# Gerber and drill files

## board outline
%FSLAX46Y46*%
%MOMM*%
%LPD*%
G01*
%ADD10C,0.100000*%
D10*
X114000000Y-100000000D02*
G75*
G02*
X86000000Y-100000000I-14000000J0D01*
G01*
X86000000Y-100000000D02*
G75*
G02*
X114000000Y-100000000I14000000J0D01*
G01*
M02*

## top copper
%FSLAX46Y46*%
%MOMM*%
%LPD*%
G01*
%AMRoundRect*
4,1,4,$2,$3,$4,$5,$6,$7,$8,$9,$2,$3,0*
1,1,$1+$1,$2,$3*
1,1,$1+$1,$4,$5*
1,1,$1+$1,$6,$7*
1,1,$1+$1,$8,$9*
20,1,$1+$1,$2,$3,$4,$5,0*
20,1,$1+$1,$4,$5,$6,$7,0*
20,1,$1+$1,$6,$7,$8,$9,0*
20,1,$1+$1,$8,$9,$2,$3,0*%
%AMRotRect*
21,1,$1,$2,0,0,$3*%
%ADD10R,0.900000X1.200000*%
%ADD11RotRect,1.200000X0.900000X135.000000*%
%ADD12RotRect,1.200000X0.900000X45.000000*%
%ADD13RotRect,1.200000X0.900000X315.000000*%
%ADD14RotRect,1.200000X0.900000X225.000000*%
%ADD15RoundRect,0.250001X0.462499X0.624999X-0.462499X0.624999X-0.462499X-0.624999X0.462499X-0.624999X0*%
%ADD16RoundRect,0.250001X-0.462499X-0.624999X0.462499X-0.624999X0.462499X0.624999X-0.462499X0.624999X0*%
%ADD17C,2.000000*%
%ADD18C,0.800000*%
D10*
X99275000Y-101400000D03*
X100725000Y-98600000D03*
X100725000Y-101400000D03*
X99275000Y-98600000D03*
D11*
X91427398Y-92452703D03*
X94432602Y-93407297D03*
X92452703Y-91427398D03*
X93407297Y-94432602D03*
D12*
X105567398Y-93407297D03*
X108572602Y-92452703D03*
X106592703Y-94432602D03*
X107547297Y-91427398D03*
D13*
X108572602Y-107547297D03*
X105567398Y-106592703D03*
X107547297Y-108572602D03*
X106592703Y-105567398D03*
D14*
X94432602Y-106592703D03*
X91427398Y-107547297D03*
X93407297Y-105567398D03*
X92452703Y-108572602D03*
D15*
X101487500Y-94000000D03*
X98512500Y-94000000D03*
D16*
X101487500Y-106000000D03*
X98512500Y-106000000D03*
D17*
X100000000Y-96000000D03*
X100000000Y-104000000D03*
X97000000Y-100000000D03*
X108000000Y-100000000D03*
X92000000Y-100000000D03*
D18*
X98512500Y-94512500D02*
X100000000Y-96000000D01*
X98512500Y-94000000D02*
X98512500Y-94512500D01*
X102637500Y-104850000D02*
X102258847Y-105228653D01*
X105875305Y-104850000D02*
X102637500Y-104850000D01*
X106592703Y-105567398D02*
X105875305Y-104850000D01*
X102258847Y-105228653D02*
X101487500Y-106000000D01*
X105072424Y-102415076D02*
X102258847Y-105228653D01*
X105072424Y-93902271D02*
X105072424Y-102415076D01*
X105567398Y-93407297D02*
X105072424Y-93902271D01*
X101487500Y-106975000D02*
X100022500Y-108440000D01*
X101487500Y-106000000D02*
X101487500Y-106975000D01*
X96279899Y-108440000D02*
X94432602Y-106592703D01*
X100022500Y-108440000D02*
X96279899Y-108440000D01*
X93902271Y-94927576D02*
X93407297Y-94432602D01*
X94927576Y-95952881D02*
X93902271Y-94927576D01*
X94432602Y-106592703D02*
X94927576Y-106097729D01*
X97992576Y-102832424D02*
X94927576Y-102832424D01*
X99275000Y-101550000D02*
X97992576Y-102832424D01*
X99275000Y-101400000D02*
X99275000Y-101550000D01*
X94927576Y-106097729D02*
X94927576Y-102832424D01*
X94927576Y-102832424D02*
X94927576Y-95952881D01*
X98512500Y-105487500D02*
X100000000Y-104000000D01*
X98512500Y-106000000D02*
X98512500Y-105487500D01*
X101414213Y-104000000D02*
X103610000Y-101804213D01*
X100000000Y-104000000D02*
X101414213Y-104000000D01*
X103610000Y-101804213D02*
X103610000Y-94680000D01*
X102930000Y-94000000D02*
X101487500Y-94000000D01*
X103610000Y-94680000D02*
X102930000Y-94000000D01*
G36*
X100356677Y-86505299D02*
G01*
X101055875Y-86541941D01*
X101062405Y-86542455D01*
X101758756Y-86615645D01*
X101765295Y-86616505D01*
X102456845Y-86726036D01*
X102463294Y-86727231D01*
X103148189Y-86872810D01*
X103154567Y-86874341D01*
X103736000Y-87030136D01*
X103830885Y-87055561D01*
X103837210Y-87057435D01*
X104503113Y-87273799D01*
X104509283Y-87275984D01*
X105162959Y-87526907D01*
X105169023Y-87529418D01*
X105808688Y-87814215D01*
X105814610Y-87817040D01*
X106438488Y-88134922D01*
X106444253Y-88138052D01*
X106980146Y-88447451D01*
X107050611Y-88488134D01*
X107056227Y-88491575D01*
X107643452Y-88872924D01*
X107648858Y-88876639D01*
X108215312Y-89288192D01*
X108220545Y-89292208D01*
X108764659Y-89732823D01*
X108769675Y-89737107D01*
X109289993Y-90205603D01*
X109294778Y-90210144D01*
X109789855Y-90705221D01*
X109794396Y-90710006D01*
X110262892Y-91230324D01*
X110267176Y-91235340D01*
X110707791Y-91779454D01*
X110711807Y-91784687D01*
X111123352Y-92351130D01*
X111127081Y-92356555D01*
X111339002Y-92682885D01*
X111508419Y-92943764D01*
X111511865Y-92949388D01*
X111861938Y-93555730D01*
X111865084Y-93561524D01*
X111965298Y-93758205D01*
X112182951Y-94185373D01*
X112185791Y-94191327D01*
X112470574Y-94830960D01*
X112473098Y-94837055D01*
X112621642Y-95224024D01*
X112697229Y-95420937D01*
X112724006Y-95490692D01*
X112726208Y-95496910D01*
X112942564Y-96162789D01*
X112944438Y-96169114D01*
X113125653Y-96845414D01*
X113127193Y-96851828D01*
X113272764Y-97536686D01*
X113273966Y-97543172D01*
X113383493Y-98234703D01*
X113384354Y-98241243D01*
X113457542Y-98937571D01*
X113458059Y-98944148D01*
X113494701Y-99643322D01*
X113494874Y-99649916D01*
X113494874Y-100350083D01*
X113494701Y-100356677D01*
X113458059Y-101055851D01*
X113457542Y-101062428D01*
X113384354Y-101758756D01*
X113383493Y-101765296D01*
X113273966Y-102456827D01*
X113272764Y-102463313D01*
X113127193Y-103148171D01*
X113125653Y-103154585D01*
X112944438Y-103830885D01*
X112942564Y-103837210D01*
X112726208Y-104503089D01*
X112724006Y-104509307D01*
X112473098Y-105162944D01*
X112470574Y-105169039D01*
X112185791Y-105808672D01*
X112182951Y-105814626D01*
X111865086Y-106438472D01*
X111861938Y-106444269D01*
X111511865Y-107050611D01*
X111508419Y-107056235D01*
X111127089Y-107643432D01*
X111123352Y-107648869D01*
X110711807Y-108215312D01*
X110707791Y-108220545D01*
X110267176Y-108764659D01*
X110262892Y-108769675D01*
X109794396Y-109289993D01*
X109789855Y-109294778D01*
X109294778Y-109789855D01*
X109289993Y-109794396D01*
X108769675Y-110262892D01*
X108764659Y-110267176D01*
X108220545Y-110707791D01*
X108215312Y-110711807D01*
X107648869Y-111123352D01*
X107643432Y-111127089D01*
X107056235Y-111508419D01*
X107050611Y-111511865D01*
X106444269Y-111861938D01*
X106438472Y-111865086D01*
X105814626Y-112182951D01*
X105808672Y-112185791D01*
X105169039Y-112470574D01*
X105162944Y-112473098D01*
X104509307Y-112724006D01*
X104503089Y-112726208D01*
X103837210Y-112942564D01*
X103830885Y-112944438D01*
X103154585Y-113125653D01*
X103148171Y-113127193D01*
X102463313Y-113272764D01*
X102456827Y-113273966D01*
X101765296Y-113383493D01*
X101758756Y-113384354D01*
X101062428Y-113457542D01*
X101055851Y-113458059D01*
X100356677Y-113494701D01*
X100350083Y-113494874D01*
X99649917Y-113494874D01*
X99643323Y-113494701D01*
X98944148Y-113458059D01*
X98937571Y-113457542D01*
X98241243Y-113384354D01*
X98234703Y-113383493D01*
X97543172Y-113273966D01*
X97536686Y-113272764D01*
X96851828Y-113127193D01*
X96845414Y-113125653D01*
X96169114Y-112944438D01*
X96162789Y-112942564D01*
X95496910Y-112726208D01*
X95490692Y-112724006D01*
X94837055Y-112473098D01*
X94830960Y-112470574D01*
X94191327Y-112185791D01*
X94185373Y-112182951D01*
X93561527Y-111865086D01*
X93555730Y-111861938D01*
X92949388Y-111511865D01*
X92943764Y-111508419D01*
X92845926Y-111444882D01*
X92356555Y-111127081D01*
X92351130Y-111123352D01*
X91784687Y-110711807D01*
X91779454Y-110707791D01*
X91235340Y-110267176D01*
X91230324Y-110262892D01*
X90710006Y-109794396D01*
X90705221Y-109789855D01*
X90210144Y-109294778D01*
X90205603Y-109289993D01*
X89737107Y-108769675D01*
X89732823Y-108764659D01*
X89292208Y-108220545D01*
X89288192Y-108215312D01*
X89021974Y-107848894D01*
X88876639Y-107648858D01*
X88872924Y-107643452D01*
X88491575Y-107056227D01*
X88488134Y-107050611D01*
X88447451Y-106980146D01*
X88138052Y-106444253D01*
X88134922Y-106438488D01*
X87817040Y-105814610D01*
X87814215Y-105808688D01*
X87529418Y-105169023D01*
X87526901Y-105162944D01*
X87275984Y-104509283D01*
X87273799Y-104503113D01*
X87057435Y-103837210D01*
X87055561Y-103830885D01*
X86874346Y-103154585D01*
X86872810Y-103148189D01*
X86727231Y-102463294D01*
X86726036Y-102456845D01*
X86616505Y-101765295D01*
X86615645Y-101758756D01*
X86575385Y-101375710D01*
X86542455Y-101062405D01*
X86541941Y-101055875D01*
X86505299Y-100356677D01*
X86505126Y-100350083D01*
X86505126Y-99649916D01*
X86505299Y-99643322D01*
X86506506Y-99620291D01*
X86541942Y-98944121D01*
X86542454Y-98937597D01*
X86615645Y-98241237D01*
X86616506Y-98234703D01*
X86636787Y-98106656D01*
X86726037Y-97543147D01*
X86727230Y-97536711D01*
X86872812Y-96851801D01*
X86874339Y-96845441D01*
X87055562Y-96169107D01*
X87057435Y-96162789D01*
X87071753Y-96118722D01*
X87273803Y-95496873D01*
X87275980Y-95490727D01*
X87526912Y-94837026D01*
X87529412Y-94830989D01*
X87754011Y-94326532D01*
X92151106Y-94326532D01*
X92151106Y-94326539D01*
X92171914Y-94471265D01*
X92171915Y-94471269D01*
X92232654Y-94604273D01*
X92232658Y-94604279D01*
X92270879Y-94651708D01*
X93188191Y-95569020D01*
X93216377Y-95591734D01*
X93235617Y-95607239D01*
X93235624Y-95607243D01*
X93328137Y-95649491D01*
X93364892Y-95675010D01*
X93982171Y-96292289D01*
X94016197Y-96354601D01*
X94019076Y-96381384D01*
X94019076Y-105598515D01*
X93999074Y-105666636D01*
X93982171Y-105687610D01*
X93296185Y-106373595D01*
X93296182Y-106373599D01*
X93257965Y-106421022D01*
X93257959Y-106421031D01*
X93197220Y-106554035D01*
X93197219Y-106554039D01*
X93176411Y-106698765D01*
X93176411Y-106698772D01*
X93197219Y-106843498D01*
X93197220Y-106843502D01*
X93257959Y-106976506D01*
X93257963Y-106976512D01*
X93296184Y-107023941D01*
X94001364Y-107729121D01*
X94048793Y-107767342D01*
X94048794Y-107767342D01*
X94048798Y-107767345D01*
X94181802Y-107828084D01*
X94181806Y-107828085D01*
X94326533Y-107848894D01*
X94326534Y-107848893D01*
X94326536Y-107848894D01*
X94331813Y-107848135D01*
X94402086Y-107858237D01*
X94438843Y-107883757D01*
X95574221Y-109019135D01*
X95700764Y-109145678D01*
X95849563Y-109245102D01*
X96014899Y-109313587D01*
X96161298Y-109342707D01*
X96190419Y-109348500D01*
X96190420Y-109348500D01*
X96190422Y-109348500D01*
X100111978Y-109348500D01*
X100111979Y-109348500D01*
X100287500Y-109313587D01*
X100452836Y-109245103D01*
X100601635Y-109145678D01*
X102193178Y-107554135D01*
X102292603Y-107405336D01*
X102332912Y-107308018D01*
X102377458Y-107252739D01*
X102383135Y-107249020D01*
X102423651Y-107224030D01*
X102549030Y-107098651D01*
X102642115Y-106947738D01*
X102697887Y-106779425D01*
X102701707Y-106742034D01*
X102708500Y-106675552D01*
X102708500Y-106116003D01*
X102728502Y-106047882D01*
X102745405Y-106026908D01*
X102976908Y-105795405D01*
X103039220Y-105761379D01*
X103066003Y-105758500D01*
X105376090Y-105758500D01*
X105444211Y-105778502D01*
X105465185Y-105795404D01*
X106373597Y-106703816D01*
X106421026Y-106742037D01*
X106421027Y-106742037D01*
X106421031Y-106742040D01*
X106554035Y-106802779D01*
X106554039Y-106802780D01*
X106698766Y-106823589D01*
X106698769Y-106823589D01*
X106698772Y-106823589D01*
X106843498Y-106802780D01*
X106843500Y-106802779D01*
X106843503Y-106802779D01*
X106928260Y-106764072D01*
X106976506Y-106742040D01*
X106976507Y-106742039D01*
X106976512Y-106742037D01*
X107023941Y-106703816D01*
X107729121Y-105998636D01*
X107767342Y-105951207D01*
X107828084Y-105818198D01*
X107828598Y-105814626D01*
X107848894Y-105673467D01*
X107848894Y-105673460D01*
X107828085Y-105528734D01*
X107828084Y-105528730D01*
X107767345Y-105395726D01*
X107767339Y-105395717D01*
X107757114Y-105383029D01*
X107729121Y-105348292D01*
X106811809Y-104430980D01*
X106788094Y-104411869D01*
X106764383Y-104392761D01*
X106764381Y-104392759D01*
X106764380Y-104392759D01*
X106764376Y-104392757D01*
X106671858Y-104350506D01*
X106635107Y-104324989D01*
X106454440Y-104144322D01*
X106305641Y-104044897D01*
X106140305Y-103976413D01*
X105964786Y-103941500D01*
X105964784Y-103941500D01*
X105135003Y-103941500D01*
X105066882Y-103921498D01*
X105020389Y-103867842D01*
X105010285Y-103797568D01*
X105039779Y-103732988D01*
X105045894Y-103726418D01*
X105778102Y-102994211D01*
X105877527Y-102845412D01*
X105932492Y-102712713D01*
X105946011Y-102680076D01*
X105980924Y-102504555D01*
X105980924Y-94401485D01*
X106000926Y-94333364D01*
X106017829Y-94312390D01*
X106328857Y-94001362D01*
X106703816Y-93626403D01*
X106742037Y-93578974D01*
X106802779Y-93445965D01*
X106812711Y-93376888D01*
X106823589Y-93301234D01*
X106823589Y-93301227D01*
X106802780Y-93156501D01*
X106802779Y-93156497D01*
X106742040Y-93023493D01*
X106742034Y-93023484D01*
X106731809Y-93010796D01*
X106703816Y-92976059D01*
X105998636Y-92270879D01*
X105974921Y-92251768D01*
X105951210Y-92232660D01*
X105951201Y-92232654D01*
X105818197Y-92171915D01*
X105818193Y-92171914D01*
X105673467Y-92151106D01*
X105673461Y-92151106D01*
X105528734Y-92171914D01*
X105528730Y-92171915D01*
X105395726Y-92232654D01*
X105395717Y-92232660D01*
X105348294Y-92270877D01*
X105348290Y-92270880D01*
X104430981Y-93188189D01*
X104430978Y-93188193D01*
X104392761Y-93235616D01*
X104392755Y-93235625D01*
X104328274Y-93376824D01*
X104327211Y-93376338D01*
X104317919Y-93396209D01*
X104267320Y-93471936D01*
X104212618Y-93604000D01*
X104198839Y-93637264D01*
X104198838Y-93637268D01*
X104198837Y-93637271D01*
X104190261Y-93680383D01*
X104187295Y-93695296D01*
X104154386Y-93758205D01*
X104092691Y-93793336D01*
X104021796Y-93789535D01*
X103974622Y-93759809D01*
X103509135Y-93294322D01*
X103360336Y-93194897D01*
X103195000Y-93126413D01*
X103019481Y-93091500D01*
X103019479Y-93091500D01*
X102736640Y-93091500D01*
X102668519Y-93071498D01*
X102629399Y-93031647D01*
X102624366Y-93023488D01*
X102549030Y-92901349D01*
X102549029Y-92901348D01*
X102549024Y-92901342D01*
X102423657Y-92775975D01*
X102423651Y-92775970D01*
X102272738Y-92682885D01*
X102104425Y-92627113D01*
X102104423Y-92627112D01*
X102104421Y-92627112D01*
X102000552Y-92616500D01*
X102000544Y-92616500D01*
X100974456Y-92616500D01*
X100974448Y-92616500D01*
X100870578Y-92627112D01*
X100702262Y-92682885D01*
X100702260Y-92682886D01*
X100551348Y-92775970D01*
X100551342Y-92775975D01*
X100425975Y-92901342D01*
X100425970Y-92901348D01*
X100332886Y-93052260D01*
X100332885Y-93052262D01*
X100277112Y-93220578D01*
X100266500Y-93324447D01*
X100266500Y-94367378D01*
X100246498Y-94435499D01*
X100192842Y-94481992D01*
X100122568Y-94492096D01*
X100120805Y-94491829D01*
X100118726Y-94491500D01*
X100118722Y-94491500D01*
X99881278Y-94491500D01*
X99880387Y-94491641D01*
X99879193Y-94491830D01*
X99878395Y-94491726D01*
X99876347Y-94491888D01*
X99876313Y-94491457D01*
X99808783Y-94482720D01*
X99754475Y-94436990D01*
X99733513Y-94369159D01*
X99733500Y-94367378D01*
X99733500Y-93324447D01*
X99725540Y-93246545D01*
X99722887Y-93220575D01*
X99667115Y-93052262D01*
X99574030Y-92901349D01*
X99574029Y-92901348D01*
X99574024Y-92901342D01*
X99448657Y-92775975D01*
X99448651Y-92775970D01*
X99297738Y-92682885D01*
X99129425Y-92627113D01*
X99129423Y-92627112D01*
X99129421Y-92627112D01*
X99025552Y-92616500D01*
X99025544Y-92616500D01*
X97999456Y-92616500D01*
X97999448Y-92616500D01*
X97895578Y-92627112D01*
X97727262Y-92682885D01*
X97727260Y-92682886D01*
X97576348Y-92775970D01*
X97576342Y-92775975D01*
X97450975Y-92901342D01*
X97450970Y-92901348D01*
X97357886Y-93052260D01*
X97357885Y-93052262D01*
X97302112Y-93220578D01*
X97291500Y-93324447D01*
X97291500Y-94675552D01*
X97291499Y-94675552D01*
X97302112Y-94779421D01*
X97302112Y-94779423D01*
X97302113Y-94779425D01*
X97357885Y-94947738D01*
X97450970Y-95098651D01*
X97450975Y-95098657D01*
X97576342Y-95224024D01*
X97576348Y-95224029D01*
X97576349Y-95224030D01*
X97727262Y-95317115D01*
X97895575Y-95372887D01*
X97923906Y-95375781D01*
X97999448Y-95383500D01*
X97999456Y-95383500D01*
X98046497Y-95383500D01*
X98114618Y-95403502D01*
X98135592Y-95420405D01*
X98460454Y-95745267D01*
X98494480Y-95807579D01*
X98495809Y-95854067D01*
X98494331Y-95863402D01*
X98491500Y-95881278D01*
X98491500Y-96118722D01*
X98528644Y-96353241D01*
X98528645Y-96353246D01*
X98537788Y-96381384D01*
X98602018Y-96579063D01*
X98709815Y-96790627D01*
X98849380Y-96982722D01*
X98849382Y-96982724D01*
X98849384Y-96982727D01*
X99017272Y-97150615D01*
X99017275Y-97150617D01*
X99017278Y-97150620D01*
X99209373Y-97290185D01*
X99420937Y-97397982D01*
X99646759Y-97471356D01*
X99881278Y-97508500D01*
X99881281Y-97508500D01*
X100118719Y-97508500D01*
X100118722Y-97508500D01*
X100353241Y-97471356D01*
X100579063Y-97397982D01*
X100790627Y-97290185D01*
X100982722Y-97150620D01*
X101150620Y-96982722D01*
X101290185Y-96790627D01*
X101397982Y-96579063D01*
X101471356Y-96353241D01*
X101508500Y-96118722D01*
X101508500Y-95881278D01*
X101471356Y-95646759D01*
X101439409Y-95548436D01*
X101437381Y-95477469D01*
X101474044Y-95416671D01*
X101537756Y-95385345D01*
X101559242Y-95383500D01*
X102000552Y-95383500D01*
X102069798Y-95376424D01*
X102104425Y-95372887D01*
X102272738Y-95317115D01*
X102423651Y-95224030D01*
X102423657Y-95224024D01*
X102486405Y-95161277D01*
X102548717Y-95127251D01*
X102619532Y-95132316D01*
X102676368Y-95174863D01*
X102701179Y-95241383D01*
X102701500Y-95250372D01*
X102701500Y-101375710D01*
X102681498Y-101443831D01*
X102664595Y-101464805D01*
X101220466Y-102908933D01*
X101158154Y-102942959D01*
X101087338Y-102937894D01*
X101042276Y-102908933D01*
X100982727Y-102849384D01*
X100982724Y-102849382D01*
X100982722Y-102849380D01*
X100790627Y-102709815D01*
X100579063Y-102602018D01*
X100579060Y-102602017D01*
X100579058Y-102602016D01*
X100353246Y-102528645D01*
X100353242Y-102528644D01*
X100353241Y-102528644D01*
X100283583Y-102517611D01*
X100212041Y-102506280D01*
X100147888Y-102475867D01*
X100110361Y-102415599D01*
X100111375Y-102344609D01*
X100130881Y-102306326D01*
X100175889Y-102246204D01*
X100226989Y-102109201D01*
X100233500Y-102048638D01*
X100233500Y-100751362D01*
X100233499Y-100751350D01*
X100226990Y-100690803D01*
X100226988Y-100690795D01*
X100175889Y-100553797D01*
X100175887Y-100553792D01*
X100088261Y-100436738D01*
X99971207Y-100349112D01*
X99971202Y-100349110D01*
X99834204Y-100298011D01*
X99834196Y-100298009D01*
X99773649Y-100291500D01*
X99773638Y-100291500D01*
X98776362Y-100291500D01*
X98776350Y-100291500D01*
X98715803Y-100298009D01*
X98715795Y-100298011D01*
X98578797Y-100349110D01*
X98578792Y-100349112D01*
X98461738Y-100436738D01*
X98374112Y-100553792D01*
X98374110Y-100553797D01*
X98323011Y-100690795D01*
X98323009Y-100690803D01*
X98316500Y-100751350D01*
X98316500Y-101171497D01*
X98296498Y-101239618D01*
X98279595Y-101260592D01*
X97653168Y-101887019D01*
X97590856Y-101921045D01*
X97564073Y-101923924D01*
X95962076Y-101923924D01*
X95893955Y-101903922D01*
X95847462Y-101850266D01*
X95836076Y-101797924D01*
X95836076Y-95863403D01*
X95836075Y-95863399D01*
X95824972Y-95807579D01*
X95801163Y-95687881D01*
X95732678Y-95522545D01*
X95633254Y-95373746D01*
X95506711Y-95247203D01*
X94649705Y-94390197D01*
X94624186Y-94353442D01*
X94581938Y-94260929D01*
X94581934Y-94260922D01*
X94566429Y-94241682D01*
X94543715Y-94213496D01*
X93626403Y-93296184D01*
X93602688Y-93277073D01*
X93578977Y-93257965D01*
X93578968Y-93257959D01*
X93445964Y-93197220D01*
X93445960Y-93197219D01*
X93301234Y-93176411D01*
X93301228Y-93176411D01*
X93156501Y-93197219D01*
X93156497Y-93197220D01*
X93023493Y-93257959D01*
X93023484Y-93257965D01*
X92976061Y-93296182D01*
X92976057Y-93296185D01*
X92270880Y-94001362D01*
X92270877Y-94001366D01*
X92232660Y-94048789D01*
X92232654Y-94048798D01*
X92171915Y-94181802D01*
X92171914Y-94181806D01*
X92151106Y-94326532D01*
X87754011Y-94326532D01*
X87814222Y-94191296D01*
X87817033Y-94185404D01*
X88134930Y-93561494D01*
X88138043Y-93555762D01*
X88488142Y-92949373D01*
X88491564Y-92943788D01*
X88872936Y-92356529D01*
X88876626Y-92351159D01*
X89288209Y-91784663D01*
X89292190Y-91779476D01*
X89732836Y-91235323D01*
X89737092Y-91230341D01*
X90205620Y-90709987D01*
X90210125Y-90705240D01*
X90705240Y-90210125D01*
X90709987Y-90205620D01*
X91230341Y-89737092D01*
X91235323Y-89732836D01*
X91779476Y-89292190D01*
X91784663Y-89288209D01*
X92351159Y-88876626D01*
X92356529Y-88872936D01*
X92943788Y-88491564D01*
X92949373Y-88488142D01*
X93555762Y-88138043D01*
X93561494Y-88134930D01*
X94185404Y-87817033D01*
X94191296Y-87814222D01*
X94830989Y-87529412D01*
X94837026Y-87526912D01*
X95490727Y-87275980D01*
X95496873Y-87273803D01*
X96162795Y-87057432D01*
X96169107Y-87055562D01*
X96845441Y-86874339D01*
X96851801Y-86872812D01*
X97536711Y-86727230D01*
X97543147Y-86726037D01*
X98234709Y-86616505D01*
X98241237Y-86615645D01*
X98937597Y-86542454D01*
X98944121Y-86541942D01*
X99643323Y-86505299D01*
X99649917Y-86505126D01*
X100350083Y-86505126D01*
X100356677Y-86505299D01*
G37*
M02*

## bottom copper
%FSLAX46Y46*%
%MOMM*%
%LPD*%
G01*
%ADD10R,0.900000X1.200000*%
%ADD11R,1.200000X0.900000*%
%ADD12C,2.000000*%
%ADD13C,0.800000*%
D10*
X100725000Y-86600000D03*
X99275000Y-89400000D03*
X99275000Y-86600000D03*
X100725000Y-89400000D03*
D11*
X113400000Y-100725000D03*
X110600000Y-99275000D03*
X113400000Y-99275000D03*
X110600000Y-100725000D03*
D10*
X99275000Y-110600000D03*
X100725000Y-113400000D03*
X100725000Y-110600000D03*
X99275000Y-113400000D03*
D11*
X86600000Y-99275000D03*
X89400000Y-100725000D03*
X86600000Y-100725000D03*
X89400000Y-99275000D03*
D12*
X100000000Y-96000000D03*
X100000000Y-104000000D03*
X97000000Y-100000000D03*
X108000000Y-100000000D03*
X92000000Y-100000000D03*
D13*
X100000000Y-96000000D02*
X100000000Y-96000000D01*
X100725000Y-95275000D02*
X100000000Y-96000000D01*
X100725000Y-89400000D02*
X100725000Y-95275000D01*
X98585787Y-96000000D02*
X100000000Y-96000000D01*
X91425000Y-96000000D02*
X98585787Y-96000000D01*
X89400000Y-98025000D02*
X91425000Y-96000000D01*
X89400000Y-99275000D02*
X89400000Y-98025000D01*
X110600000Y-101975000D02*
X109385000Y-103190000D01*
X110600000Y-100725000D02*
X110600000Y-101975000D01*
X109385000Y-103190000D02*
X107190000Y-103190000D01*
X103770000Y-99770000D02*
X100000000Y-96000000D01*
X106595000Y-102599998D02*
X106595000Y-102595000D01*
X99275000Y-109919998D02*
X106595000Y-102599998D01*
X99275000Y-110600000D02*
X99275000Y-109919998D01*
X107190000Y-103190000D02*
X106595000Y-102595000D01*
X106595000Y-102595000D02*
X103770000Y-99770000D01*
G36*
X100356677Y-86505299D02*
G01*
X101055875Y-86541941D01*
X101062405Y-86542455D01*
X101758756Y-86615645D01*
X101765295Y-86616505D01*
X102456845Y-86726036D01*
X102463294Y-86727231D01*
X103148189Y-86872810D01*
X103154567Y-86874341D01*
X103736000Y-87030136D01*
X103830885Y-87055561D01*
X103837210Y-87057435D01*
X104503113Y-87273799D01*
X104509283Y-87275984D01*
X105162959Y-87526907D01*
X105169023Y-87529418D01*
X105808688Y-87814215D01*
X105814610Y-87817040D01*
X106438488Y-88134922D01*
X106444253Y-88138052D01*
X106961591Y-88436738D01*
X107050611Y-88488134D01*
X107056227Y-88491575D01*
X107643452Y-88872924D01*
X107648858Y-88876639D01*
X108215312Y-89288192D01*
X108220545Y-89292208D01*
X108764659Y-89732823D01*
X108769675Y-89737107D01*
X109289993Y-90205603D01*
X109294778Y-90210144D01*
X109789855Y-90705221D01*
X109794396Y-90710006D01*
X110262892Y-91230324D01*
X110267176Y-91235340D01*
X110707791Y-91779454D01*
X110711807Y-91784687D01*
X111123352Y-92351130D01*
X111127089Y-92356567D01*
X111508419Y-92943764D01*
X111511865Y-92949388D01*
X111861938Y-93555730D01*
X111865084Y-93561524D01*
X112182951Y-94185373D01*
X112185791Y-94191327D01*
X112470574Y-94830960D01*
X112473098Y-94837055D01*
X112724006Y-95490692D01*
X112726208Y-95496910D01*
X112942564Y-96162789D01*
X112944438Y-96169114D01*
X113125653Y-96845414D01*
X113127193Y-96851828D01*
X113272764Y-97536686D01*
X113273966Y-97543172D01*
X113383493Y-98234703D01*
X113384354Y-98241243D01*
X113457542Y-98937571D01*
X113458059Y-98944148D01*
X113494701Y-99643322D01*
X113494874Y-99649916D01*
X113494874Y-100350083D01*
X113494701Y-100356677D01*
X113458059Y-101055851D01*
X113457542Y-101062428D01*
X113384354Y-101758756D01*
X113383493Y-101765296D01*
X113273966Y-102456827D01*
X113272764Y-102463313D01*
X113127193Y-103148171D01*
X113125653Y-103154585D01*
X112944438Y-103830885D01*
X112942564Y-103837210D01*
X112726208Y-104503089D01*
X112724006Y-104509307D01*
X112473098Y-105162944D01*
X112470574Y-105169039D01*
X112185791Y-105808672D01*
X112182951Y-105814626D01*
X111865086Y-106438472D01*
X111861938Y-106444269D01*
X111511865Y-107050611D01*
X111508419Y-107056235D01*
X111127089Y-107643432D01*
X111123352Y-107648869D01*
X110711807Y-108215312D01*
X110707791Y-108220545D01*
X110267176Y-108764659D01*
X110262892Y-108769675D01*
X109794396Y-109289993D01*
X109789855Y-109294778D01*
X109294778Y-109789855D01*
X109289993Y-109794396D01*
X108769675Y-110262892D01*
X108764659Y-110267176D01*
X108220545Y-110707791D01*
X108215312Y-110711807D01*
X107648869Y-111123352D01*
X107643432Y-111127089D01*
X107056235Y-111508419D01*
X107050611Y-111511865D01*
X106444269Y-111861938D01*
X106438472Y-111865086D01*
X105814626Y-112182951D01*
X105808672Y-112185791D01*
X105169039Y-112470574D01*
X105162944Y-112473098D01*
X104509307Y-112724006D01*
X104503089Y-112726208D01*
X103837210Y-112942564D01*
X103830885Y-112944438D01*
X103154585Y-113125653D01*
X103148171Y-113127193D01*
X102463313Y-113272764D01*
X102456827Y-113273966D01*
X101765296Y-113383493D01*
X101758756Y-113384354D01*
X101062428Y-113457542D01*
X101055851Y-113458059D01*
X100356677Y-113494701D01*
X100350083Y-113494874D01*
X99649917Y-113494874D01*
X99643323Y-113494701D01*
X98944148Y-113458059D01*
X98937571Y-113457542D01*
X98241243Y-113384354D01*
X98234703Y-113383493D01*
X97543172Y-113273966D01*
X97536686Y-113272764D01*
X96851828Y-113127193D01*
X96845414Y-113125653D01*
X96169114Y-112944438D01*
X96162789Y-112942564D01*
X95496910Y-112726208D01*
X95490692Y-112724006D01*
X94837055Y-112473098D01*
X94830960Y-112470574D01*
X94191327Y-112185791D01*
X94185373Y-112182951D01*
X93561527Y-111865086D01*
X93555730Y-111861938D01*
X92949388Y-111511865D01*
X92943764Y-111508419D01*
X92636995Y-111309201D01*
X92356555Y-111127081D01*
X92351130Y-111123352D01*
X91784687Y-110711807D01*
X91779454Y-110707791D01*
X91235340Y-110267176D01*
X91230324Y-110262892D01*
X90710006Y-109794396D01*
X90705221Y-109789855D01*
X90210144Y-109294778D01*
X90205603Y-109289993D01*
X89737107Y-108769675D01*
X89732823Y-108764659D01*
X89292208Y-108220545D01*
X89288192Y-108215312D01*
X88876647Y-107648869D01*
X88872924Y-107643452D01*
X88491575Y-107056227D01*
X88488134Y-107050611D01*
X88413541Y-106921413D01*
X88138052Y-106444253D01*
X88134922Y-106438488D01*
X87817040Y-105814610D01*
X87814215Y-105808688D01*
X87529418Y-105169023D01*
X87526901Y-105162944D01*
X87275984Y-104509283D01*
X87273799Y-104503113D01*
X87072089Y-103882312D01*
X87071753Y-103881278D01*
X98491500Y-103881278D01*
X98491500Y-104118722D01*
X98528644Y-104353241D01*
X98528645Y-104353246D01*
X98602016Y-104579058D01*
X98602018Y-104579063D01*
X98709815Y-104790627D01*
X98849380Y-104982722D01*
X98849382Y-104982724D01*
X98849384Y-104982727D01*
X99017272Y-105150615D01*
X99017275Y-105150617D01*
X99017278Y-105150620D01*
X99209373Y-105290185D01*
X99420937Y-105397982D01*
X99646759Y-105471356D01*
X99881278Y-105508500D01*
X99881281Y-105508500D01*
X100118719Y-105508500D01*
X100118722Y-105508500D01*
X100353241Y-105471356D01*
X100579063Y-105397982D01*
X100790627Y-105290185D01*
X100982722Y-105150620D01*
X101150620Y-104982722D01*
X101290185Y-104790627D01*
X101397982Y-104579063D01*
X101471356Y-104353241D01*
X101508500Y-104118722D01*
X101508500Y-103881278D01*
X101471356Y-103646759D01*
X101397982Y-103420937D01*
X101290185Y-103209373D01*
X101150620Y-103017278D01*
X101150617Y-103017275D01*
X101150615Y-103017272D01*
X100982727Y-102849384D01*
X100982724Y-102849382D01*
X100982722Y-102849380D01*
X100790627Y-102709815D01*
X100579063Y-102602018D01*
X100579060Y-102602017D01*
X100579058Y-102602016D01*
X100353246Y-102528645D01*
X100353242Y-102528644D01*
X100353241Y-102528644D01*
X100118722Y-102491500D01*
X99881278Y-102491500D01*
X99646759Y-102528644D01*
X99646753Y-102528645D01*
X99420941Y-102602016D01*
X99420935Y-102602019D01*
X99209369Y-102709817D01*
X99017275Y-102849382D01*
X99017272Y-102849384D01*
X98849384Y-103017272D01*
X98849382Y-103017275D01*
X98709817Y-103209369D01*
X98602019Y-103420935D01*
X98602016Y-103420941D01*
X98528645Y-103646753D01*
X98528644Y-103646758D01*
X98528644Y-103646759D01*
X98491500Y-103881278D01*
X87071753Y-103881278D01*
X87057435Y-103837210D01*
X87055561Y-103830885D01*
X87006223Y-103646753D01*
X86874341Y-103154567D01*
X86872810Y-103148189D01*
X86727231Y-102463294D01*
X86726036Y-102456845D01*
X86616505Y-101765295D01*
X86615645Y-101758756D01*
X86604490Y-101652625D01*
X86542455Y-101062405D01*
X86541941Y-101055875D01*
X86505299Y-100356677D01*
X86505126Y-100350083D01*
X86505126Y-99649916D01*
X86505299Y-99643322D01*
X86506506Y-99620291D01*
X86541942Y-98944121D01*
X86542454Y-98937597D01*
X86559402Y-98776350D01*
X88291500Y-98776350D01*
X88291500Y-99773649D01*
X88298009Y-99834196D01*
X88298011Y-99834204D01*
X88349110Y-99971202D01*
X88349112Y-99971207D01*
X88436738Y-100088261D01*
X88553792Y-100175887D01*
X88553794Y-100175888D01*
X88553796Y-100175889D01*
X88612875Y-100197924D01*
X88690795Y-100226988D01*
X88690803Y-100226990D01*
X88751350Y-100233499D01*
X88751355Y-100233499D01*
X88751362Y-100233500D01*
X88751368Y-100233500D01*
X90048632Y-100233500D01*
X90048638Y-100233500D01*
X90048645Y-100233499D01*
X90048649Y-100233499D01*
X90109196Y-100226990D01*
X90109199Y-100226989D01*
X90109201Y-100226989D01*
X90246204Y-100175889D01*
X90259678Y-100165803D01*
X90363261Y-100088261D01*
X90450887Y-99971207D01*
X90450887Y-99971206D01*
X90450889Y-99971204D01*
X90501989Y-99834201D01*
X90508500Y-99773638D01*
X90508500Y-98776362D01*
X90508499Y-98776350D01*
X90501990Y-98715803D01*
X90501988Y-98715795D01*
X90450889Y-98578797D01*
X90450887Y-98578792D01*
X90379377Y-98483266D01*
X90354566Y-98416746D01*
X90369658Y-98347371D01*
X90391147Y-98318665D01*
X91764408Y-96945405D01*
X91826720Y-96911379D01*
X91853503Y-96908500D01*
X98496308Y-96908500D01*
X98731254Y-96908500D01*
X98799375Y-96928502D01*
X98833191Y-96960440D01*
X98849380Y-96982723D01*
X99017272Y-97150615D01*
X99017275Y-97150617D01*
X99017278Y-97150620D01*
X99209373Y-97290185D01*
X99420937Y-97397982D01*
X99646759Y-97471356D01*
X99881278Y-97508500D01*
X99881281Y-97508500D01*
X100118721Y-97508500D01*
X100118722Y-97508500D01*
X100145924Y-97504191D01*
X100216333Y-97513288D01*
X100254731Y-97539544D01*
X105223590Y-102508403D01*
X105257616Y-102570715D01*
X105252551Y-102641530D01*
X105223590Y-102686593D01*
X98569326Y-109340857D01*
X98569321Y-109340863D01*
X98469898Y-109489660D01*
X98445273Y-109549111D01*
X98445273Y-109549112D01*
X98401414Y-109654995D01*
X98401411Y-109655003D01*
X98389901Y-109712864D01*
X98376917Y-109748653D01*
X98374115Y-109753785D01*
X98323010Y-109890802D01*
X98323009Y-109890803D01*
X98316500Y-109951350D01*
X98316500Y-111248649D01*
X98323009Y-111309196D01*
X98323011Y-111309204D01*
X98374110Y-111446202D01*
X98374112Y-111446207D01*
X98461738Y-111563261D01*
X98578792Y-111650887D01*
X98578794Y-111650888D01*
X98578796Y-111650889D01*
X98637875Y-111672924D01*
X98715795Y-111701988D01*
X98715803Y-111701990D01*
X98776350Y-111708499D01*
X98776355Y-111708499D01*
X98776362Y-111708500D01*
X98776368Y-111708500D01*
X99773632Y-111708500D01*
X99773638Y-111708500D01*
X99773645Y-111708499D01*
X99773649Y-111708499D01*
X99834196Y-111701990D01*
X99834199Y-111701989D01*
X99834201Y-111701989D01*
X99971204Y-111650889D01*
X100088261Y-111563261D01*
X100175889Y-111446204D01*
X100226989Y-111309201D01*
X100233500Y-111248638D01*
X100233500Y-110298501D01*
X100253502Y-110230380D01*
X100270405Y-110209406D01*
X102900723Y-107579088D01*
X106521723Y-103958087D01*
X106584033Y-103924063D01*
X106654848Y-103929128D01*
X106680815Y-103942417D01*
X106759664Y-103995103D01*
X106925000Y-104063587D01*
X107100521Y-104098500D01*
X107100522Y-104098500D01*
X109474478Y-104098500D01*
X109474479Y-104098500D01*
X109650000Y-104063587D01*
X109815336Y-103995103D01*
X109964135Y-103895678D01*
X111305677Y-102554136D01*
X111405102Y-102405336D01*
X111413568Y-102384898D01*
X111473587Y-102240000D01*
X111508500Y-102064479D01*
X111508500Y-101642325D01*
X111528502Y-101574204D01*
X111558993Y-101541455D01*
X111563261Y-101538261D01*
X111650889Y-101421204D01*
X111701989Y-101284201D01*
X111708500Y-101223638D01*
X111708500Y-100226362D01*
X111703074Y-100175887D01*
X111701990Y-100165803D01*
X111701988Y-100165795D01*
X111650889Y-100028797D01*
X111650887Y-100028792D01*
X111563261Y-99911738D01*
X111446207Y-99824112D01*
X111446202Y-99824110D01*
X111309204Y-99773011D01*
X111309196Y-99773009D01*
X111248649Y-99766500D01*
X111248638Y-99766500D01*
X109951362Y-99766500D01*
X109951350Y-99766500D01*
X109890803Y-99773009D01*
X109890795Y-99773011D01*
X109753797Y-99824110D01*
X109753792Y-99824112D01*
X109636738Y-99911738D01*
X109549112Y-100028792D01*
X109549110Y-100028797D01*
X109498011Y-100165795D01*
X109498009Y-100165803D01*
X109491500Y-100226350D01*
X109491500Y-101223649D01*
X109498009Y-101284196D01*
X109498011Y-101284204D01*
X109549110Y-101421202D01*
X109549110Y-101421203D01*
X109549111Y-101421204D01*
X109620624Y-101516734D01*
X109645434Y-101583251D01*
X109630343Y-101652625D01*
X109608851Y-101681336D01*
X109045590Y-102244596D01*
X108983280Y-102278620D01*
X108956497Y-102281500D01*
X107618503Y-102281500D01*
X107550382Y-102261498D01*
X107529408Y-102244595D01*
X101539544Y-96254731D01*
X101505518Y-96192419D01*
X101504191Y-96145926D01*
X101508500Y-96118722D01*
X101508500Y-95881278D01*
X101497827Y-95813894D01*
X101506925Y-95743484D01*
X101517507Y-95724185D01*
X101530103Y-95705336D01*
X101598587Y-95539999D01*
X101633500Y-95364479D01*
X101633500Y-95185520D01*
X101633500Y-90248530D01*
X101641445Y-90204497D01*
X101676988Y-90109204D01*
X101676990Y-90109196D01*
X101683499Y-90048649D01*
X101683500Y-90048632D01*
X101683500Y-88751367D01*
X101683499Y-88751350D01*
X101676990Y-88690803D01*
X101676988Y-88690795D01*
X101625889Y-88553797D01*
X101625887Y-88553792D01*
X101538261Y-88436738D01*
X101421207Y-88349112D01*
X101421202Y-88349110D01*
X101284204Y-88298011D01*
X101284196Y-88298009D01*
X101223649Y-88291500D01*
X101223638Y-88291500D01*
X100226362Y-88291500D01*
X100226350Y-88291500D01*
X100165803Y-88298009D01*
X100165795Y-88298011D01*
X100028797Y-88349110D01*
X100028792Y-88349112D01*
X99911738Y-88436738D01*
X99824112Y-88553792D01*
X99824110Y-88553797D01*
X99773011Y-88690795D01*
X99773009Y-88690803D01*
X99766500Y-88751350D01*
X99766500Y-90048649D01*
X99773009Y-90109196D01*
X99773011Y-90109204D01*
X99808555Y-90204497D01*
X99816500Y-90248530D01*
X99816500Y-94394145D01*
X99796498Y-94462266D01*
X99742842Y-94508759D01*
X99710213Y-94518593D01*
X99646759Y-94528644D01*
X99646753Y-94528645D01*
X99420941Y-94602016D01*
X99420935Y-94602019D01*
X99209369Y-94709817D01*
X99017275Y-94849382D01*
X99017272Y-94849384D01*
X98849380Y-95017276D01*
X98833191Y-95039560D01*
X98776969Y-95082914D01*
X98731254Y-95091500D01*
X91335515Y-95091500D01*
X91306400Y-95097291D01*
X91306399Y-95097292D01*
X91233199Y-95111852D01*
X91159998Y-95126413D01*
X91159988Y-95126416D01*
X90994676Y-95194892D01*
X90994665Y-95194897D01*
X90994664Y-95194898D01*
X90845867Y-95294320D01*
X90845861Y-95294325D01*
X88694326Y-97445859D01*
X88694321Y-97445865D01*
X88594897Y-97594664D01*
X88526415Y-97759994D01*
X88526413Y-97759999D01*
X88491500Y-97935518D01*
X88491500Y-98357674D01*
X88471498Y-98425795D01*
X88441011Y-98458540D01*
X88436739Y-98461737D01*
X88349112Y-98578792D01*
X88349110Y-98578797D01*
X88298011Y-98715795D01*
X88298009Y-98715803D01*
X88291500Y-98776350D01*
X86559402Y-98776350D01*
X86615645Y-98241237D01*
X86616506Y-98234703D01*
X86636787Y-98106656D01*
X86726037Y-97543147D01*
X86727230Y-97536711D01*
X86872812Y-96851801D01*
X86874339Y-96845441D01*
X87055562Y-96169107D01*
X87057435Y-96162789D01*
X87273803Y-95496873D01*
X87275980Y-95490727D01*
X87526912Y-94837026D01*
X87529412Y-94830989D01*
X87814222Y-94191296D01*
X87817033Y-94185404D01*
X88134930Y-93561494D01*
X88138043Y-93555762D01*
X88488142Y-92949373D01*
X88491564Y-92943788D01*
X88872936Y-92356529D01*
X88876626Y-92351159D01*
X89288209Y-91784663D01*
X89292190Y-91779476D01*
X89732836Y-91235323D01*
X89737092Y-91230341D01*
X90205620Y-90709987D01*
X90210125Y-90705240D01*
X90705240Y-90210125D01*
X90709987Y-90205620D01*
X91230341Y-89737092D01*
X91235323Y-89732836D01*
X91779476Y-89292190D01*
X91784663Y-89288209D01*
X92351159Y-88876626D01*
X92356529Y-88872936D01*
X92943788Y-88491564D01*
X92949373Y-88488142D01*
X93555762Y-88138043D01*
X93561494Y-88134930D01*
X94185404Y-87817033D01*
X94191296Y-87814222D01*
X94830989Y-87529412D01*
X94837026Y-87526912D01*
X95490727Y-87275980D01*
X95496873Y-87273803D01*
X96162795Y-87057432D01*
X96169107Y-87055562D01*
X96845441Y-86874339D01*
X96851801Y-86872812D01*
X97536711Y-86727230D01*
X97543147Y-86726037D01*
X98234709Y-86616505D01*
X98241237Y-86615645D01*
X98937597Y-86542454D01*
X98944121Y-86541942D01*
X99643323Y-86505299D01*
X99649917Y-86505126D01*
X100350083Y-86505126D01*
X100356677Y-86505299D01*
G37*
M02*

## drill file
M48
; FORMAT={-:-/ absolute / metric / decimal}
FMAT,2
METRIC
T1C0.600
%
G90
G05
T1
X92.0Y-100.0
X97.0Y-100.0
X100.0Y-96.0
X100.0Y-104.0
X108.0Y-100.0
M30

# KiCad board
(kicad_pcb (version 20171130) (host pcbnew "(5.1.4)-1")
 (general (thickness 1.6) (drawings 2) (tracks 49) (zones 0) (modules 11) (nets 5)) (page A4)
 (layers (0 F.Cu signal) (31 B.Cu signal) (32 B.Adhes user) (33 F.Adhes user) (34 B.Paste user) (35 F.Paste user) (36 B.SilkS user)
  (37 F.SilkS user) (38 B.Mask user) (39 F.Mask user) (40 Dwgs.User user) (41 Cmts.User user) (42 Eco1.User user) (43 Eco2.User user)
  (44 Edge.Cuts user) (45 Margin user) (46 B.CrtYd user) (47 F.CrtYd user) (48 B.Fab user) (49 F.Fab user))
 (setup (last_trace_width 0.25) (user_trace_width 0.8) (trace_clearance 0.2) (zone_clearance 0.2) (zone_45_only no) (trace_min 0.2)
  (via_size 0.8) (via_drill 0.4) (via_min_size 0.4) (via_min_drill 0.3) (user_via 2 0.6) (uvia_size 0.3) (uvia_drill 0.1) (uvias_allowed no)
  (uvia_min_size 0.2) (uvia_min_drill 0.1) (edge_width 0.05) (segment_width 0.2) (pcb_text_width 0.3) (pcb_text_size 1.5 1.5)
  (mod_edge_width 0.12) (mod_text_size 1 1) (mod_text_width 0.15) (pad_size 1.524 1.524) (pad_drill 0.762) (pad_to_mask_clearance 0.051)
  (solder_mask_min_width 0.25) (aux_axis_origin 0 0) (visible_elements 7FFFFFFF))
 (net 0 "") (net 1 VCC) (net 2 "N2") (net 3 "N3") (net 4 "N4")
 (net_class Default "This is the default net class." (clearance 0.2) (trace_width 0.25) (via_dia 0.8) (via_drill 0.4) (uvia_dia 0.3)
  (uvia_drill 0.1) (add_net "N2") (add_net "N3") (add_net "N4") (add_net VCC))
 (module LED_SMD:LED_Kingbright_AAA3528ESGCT (layer B.Cu) (at 100 88 90)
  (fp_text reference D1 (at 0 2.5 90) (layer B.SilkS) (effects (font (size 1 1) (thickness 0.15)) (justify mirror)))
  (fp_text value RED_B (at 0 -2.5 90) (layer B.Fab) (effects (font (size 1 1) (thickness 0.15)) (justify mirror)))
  (pad 2 smd rect (at 1.4 0.725 90) (size 1.2 0.9) (layers B.Cu B.Paste B.Mask) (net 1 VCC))
  (pad 4 smd rect (at -1.4 -0.725 90) (size 1.2 0.9) (layers B.Cu B.Paste B.Mask) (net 1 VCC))
  (pad 3 smd rect (at 1.4 -0.725 90) (size 1.2 0.9) (layers B.Cu B.Paste B.Mask) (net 1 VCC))
  (pad 1 smd rect (at -1.4 0.725 90) (size 1.2 0.9) (layers B.Cu B.Paste B.Mask) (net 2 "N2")))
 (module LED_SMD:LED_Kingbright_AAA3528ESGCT (layer B.Cu) (at 112 100)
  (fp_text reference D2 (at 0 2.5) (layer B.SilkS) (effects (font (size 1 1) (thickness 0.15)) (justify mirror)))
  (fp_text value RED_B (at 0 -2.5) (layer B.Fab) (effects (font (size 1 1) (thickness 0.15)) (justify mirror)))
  (pad 2 smd rect (at 1.4 0.725) (size 1.2 0.9) (layers B.Cu B.Paste B.Mask) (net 1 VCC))
  (pad 4 smd rect (at -1.4 -0.725) (size 1.2 0.9) (layers B.Cu B.Paste B.Mask) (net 1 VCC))
  (pad 3 smd rect (at 1.4 -0.725) (size 1.2 0.9) (layers B.Cu B.Paste B.Mask) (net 1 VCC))
  (pad 1 smd rect (at -1.4 0.725) (size 1.2 0.9) (layers B.Cu B.Paste B.Mask) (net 2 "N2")))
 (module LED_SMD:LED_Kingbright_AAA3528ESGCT (layer B.Cu) (at 100 112 270)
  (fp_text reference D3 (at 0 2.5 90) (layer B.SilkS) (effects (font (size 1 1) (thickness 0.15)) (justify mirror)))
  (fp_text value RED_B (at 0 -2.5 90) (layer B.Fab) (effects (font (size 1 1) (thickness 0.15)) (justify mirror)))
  (pad 1 smd rect (at -1.4 0.725 270) (size 1.2 0.9) (layers B.Cu B.Paste B.Mask) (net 2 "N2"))
  (pad 3 smd rect (at 1.4 -0.725 270) (size 1.2 0.9) (layers B.Cu B.Paste B.Mask) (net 1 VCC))
  (pad 4 smd rect (at -1.4 -0.725 270) (size 1.2 0.9) (layers B.Cu B.Paste B.Mask) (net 1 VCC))
  (pad 2 smd rect (at 1.4 0.725 270) (size 1.2 0.9) (layers B.Cu B.Paste B.Mask) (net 1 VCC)))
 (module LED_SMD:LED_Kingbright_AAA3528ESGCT (layer B.Cu) (at 88 100 180)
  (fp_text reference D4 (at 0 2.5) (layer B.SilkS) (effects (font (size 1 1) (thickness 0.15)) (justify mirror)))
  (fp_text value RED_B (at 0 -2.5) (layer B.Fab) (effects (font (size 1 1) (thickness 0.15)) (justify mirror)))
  (pad 2 smd rect (at 1.4 0.725 180) (size 1.2 0.9) (layers B.Cu B.Paste B.Mask) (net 1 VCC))
  (pad 4 smd rect (at -1.4 -0.725 180) (size 1.2 0.9) (layers B.Cu B.Paste B.Mask) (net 1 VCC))
  (pad 3 smd rect (at 1.4 -0.725 180) (size 1.2 0.9) (layers B.Cu B.Paste B.Mask) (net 1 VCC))
  (pad 1 smd rect (at -1.4 0.725 180) (size 1.2 0.9) (layers B.Cu B.Paste B.Mask) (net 2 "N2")))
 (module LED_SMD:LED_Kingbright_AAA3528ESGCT (layer F.Cu) (at 100 100 90)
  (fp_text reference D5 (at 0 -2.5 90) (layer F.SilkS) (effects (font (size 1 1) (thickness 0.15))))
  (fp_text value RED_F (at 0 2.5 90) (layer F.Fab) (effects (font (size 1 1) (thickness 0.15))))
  (pad 1 smd rect (at -1.4 -0.725 90) (size 1.2 0.9) (layers F.Cu F.Paste F.Mask) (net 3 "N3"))
  (pad 3 smd rect (at 1.4 0.725 90) (size 1.2 0.9) (layers F.Cu F.Paste F.Mask) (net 1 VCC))
  (pad 4 smd rect (at -1.4 0.725 90) (size 1.2 0.9) (layers F.Cu F.Paste F.Mask) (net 1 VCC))
  (pad 2 smd rect (at 1.4 -0.725 90) (size 1.2 0.9) (layers F.Cu F.Paste F.Mask) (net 1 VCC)))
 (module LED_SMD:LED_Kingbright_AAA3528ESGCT (layer F.Cu) (at 92.93 92.93 135)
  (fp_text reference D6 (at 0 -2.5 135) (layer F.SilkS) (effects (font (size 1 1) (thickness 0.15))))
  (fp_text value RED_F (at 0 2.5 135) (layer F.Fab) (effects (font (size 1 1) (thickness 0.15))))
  (pad 2 smd rect (at 1.4 -0.725 135) (size 1.2 0.9) (layers F.Cu F.Paste F.Mask) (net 1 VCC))
  (pad 4 smd rect (at -1.4 0.725 135) (size 1.2 0.9) (layers F.Cu F.Paste F.Mask) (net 1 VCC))
  (pad 3 smd rect (at 1.4 0.725 135) (size 1.2 0.9) (layers F.Cu F.Paste F.Mask) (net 1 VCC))
  (pad 1 smd rect (at -1.4 -0.725 135) (size 1.2 0.9) (layers F.Cu F.Paste F.Mask) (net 3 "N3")))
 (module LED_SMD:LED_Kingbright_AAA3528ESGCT (layer F.Cu) (at 107.07 92.93 45)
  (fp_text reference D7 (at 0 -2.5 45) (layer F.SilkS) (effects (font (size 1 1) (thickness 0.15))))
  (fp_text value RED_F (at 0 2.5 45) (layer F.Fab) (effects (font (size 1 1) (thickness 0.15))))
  (pad 1 smd rect (at -1.4 -0.725 45) (size 1.2 0.9) (layers F.Cu F.Paste F.Mask) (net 3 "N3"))
  (pad 3 smd rect (at 1.4 0.725 45) (size 1.2 0.9) (layers F.Cu F.Paste F.Mask) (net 1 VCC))
  (pad 4 smd rect (at -1.4 0.725 45) (size 1.2 0.9) (layers F.Cu F.Paste F.Mask) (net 1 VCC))
  (pad 2 smd rect (at 1.4 -0.725 45) (size 1.2 0.9) (layers F.Cu F.Paste F.Mask) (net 1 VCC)))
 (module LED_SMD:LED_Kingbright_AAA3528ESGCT (layer F.Cu) (at 107.07 107.07 315)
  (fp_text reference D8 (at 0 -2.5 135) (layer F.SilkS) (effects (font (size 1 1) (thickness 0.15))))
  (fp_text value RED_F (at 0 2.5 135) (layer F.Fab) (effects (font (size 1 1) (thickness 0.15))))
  (pad 2 smd rect (at 1.4 -0.725 315) (size 1.2 0.9) (layers F.Cu F.Paste F.Mask) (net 1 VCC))
  (pad 4 smd rect (at -1.4 0.725 315) (size 1.2 0.9) (layers F.Cu F.Paste F.Mask) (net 1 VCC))
  (pad 3 smd rect (at 1.4 0.725 315) (size 1.2 0.9) (layers F.Cu F.Paste F.Mask) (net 1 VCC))
  (pad 1 smd rect (at -1.4 -0.725 315) (size 1.2 0.9) (layers F.Cu F.Paste F.Mask) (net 3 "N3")))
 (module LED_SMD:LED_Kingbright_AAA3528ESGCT (layer F.Cu) (at 92.93 107.07 225)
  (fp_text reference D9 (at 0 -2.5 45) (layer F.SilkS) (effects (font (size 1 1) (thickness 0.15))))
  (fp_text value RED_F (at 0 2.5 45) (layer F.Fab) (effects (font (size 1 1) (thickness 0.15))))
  (pad 1 smd rect (at -1.4 -0.725 225) (size 1.2 0.9) (layers F.Cu F.Paste F.Mask) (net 3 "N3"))
  (pad 3 smd rect (at 1.4 0.725 225) (size 1.2 0.9) (layers F.Cu F.Paste F.Mask) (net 1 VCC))
  (pad 4 smd rect (at -1.4 0.725 225) (size 1.2 0.9) (layers F.Cu F.Paste F.Mask) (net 1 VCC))
  (pad 2 smd rect (at 1.4 -0.725 225) (size 1.2 0.9) (layers F.Cu F.Paste F.Mask) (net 1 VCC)))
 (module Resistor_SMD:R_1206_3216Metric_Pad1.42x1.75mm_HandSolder (layer F.Cu) (at 100 94 180)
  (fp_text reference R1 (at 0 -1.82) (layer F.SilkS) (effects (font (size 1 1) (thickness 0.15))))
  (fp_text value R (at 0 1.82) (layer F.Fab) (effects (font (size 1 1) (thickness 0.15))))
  (pad 1 smd roundrect (at -1.4875 0 180) (size 1.425 1.75) (layers F.Cu F.Paste F.Mask) (roundrect_rratio 0.175439) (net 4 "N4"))
  (pad 2 smd roundrect (at 1.4875 0 180) (size 1.425 1.75) (layers F.Cu F.Paste F.Mask) (roundrect_rratio 0.175439) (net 2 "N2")))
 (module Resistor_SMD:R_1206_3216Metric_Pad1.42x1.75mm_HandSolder (layer F.Cu) (at 100 106)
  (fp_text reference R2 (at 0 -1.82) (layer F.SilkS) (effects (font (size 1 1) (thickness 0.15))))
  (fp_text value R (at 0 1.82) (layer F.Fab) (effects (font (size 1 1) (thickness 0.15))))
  (pad 2 smd roundrect (at 1.4875 0) (size 1.425 1.75) (layers F.Cu F.Paste F.Mask) (roundrect_rratio 0.175439) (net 3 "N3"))
  (pad 1 smd roundrect (at -1.4875 0) (size 1.425 1.75) (layers F.Cu F.Paste F.Mask) (roundrect_rratio 0.175439) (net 4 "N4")))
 (gr_circle (center 100 100) (end 114 100) (layer Edge.Cuts) (width 0.1))
 (segment (start 100 96) (end 100 96) (width 0.8) (layer B.Cu) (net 2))
 (via (at 100 96) (size 2) (drill 0.6) (layers F.Cu B.Cu) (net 2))
 (segment (start 100.725 95.275) (end 100 96) (width 0.8) (layer B.Cu) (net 2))
 (segment (start 100.725 89.4) (end 100.725 95.275) (width 0.8) (layer B.Cu) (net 2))
 (segment (start 98.5125 94.5125) (end 100 96) (width 0.8) (layer F.Cu) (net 2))
 (segment (start 98.5125 94) (end 98.5125 94.5125) (width 0.8) (layer F.Cu) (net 2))
 (segment (start 98.585787 96) (end 100 96) (width 0.8) (layer B.Cu) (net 2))
 (segment (start 91.425 96) (end 98.585787 96) (width 0.8) (layer B.Cu) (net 2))
 (segment (start 89.4 98.025) (end 91.425 96) (width 0.8) (layer B.Cu) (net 2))
 (segment (start 89.4 99.275) (end 89.4 98.025) (width 0.8) (layer B.Cu) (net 2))
 (segment (start 110.6 101.975) (end 109.385 103.19) (width 0.8) (layer B.Cu) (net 2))
 (segment (start 110.6 100.725) (end 110.6 101.975) (width 0.8) (layer B.Cu) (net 2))
 (segment (start 109.385 103.19) (end 107.19 103.19) (width 0.8) (layer B.Cu) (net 2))
 (segment (start 103.77 99.77) (end 100 96) (width 0.8) (layer B.Cu) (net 2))
 (segment (start 106.595 102.599998) (end 106.595 102.595) (width 0.8) (layer B.Cu) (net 2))
 (segment (start 99.275 109.919998) (end 106.595 102.599998) (width 0.8) (layer B.Cu) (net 2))
 (segment (start 99.275 110.6) (end 99.275 109.919998) (width 0.8) (layer B.Cu) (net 2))
 (segment (start 107.19 103.19) (end 106.595 102.595) (width 0.8) (layer B.Cu) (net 2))
 (segment (start 106.595 102.595) (end 103.77 99.77) (width 0.8) (layer B.Cu) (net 2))
 (segment (start 102.6375 104.85) (end 102.258847 105.228653) (width 0.8) (layer F.Cu) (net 3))
 (segment (start 105.875305 104.85) (end 102.6375 104.85) (width 0.8) (layer F.Cu) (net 3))
 (segment (start 106.592703 105.567398) (end 105.875305 104.85) (width 0.8) (layer F.Cu) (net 3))
 (segment (start 102.258847 105.228653) (end 101.4875 106) (width 0.8) (layer F.Cu) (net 3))
 (segment (start 105.072424 102.415076) (end 102.258847 105.228653) (width 0.8) (layer F.Cu) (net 3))
 (segment (start 105.072424 93.902271) (end 105.072424 102.415076) (width 0.8) (layer F.Cu) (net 3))
 (segment (start 105.567398 93.407297) (end 105.072424 93.902271) (width 0.8) (layer F.Cu) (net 3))
 (segment (start 101.4875 106.975) (end 100.0225 108.44) (width 0.8) (layer F.Cu) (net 3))
 (segment (start 101.4875 106) (end 101.4875 106.975) (width 0.8) (layer F.Cu) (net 3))
 (segment (start 96.279899 108.44) (end 94.432602 106.592703) (width 0.8) (layer F.Cu) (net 3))
 (segment (start 100.0225 108.44) (end 96.279899 108.44) (width 0.8) (layer F.Cu) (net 3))
 (segment (start 93.902271 94.927576) (end 93.407297 94.432602) (width 0.8) (layer F.Cu) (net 3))
 (segment (start 94.927576 95.952881) (end 93.902271 94.927576) (width 0.8) (layer F.Cu) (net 3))
 (segment (start 94.432602 106.592703) (end 94.927576 106.097729) (width 0.8) (layer F.Cu) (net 3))
 (segment (start 97.992576 102.832424) (end 94.927576 102.832424) (width 0.8) (layer F.Cu) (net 3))
 (segment (start 99.275 101.55) (end 97.992576 102.832424) (width 0.8) (layer F.Cu) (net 3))
 (segment (start 99.275 101.4) (end 99.275 101.55) (width 0.8) (layer F.Cu) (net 3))
 (segment (start 94.927576 106.097729) (end 94.927576 102.832424) (width 0.8) (layer F.Cu) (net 3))
 (segment (start 94.927576 102.832424) (end 94.927576 95.952881) (width 0.8) (layer F.Cu) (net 3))
 (via (at 100 104) (size 2) (drill 0.6) (layers F.Cu B.Cu) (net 4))
 (segment (start 98.5125 105.4875) (end 100 104) (width 0.8) (layer F.Cu) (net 4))
 (segment (start 98.5125 106) (end 98.5125 105.4875) (width 0.8) (layer F.Cu) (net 4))
 (segment (start 101.414213 104) (end 103.61 101.804213) (width 0.8) (layer F.Cu) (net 4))
 (segment (start 100 104) (end 101.414213 104) (width 0.8) (layer F.Cu) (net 4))
 (segment (start 103.61 101.804213) (end 103.61 94.68) (width 0.8) (layer F.Cu) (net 4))
 (segment (start 102.93 94) (end 101.4875 94) (width 0.8) (layer F.Cu) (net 4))
 (segment (start 103.61 94.68) (end 102.93 94) (width 0.8) (layer F.Cu) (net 4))
 (via (at 97 100) (size 2) (drill 0.6) (layers F.Cu B.Cu) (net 1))
 (via (at 108 100) (size 2) (drill 0.6) (layers F.Cu B.Cu) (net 1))
 (via (at 92 100) (size 2) (drill 0.6) (layers F.Cu B.Cu) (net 1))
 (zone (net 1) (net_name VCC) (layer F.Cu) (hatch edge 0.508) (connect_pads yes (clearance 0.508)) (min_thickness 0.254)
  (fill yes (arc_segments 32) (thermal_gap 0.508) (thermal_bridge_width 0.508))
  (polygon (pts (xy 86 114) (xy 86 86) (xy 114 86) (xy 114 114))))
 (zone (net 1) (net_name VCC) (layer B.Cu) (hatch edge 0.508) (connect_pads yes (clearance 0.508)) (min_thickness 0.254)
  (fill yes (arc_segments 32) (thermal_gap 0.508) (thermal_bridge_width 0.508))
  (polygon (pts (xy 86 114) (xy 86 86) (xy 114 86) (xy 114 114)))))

